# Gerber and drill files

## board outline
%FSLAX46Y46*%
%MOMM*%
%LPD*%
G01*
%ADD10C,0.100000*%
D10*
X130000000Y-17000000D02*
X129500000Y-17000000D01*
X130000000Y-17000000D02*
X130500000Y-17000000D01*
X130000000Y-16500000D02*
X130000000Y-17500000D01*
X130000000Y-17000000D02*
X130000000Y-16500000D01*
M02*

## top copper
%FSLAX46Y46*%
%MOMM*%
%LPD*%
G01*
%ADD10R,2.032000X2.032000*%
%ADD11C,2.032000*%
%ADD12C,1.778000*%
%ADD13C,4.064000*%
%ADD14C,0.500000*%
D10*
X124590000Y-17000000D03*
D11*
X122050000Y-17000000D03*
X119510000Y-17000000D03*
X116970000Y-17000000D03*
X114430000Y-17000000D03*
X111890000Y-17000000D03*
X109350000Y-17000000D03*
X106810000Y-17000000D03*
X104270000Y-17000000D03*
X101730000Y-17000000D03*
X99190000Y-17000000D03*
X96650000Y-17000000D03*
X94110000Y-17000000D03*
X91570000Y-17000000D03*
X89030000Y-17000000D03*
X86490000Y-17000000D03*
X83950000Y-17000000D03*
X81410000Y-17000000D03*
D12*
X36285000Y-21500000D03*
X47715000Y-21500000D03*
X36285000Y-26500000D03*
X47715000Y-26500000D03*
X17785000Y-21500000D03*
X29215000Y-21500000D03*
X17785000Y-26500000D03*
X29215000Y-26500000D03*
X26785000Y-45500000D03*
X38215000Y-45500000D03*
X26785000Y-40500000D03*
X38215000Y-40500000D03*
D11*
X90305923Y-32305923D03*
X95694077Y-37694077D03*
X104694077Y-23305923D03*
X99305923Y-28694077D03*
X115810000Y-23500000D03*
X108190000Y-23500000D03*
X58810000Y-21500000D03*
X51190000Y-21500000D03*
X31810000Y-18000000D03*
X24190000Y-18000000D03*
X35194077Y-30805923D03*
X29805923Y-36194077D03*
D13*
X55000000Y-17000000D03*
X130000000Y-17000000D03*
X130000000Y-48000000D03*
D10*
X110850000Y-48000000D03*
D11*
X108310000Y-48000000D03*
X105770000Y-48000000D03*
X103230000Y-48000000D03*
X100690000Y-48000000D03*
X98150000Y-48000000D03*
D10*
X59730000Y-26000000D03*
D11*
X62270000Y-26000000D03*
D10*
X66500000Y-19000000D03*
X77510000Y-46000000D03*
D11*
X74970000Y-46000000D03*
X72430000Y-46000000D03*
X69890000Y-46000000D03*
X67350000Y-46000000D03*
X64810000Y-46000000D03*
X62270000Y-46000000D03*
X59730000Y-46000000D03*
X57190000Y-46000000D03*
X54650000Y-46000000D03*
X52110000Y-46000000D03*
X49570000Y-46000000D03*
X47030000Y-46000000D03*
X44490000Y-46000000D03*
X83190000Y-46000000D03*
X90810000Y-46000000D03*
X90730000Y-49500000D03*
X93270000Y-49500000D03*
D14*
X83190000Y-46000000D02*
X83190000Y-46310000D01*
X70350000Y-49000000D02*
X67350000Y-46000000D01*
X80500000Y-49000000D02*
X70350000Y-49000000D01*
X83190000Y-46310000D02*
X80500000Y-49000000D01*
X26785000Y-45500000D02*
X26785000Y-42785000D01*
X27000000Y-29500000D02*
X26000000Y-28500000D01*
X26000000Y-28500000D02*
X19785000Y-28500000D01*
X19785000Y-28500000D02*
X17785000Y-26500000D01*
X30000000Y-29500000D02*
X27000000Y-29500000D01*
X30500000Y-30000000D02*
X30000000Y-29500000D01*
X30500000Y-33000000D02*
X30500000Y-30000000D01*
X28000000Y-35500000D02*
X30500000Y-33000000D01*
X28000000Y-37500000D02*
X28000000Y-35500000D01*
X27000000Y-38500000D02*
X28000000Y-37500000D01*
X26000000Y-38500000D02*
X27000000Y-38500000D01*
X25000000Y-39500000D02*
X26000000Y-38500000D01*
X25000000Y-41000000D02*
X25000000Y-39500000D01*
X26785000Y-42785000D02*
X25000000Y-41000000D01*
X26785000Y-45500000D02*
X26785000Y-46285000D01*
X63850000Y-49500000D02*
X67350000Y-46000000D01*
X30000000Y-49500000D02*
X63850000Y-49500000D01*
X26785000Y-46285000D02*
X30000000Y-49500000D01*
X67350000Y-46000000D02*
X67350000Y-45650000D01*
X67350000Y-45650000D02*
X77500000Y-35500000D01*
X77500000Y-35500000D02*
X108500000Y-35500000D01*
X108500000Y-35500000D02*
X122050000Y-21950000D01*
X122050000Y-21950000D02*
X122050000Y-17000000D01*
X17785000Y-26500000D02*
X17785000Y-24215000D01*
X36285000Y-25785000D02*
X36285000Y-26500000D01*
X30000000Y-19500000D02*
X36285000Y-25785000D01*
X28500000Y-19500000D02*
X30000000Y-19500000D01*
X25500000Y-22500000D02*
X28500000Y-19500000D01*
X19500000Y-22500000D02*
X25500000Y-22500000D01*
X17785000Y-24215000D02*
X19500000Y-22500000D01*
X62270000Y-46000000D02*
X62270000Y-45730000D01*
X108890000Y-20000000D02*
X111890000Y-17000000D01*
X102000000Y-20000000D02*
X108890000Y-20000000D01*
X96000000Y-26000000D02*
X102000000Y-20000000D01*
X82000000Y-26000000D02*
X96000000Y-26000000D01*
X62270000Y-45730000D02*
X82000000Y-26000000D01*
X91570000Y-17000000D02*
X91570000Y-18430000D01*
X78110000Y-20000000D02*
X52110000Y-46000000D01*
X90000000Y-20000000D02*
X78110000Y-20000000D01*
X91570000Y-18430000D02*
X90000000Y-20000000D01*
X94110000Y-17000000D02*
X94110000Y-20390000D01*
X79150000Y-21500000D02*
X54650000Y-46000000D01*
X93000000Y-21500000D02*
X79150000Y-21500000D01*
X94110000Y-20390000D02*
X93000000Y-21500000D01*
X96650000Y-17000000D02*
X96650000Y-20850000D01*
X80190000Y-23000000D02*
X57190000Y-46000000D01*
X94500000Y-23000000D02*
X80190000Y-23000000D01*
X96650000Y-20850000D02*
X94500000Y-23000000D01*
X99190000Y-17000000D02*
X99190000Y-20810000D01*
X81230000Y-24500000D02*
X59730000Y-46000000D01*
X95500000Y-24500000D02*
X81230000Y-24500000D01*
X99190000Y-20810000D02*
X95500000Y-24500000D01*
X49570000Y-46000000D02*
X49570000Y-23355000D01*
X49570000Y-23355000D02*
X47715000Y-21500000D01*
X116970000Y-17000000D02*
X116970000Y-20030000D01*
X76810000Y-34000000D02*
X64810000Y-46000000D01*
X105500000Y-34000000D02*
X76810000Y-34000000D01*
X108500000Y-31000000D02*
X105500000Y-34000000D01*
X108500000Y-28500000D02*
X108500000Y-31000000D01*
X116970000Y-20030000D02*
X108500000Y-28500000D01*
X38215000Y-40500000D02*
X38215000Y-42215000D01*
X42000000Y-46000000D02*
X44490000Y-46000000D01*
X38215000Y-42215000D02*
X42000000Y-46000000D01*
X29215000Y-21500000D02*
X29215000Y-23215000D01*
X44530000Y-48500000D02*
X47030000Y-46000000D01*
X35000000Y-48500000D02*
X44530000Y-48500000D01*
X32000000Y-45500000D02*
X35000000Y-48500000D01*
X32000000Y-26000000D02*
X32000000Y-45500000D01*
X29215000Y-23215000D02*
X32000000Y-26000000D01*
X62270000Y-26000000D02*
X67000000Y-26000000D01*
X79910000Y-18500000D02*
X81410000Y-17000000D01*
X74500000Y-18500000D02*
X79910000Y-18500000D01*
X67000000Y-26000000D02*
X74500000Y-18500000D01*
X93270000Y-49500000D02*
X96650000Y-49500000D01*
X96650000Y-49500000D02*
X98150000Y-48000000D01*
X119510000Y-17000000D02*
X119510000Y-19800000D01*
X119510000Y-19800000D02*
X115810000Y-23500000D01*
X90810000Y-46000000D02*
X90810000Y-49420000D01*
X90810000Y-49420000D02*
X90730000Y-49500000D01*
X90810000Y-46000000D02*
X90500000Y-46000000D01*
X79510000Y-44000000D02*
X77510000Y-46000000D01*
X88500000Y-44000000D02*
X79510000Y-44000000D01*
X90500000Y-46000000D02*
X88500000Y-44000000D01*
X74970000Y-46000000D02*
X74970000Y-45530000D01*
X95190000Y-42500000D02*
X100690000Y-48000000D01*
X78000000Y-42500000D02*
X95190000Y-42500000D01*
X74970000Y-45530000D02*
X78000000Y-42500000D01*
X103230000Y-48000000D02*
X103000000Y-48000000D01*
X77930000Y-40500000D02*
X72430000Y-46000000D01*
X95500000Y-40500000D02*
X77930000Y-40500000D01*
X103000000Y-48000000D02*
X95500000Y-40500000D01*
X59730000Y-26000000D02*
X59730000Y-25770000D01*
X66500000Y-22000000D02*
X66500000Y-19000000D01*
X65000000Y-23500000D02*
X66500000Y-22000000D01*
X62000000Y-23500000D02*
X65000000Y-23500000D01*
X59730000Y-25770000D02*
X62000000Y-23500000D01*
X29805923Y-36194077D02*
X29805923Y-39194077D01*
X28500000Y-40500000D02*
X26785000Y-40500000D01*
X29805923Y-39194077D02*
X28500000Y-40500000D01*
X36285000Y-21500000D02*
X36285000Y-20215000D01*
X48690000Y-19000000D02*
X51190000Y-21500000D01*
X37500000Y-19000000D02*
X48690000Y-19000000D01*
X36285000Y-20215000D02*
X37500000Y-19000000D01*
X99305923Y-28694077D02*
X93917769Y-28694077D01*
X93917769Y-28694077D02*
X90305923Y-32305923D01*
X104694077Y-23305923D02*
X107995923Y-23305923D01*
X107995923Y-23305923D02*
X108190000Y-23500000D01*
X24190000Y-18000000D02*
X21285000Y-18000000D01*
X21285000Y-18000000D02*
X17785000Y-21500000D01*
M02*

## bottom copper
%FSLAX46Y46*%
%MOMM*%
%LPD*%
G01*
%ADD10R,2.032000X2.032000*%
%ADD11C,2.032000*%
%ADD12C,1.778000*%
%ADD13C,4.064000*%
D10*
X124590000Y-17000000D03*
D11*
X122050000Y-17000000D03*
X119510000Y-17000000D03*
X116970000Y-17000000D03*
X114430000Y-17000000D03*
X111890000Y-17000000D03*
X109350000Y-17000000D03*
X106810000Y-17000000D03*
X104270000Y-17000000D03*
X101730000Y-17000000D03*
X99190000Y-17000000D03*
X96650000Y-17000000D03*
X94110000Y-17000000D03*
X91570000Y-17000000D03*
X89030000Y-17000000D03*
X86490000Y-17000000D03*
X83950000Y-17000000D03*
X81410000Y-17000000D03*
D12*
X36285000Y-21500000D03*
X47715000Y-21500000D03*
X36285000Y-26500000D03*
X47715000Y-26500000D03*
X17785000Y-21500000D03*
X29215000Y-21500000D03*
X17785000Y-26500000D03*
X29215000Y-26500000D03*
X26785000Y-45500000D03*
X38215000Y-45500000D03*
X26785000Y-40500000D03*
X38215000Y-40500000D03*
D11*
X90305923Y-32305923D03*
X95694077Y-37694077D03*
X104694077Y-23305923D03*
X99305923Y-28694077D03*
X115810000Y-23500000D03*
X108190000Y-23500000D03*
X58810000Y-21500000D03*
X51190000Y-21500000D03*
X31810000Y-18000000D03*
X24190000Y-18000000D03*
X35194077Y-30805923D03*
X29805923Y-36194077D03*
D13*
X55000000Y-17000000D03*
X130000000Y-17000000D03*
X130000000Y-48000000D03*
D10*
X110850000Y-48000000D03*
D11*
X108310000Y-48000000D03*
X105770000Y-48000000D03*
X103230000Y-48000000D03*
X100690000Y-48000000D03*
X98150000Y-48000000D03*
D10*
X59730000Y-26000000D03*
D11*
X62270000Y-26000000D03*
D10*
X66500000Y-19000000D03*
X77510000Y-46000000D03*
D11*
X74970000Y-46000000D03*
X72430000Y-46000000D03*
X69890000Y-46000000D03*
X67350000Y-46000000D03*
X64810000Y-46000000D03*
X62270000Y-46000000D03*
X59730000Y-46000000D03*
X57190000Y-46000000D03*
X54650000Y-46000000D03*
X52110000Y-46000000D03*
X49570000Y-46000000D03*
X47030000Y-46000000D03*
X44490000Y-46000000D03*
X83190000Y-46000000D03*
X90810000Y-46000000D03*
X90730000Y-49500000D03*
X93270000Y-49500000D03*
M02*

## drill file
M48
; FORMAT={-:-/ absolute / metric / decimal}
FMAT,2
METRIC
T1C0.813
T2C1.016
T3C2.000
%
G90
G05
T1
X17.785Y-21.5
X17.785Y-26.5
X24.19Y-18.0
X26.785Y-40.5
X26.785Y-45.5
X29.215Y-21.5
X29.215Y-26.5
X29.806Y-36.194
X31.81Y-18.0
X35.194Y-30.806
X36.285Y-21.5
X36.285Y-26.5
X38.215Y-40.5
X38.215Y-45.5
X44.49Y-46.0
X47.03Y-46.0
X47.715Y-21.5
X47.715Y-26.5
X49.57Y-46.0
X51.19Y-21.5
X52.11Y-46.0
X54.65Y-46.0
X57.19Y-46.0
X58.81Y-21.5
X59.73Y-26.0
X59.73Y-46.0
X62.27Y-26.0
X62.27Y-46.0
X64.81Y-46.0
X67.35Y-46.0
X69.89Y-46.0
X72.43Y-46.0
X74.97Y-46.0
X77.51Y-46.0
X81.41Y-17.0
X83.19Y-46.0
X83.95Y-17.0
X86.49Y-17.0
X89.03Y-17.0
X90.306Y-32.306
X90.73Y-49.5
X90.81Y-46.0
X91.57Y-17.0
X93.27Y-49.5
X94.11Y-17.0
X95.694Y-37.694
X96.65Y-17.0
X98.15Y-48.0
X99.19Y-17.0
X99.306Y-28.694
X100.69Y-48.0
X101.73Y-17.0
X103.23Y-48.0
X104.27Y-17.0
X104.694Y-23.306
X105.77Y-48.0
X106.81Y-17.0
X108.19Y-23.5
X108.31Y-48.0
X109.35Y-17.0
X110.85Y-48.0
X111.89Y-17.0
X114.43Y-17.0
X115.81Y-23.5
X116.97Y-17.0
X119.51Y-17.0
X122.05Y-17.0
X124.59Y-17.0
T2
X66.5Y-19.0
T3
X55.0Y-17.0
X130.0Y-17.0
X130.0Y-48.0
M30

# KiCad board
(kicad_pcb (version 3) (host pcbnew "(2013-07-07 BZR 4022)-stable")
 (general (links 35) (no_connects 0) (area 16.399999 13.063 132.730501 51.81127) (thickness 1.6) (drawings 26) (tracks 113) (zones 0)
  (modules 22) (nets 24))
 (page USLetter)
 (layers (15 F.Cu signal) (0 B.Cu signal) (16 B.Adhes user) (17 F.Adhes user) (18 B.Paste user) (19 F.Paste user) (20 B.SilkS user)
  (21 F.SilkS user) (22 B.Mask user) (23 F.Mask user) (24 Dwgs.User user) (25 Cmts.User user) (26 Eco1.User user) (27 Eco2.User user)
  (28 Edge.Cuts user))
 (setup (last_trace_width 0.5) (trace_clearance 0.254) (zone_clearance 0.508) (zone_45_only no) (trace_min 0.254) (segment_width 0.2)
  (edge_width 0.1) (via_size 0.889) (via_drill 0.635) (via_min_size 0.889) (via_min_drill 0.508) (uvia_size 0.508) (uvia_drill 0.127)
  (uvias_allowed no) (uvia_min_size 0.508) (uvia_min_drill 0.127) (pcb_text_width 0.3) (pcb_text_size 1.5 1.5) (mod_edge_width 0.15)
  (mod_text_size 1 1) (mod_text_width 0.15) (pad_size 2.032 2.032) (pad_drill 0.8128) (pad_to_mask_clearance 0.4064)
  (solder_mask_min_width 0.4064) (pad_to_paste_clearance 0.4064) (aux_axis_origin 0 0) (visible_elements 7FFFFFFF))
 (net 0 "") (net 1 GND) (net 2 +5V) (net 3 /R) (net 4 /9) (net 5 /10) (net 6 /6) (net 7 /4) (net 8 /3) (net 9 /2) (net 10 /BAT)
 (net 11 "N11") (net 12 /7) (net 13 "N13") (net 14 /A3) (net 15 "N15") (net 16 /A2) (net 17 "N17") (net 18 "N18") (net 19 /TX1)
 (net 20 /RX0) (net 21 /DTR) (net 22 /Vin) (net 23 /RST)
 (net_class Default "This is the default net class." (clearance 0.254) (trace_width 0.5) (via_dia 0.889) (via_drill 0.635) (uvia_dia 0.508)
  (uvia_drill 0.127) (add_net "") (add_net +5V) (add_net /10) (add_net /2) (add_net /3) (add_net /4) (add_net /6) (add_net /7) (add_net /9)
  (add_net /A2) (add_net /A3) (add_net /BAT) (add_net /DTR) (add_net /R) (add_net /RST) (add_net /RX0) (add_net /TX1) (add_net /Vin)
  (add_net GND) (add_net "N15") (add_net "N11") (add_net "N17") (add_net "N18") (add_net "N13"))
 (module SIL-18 (layer F.Cu) (at 103 17 180) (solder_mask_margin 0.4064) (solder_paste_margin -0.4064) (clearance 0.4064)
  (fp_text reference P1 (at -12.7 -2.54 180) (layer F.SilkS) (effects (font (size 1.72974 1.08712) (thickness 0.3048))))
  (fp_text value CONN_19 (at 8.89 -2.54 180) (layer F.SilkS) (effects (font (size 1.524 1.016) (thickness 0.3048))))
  (pad 1 thru_hole rect (at -21.59 0 180) (size 2.032 2.032) (drill 0.8128) (layers *.Cu *.Mask F.SilkS) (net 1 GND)
   (solder_mask_margin 0.4064) (solder_paste_margin -0.4064) (clearance 0.4064) (thermal_width 0.508) (thermal_gap 0.508))
  (pad 2 thru_hole circle (at -19.05 0 180) (size 2.032 2.032) (drill 0.8128) (layers *.Cu *.Mask F.SilkS) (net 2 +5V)
   (solder_mask_margin 0.4064) (solder_paste_margin -0.4064))
  (pad 3 thru_hole circle (at -16.51 0 180) (size 2.032 2.032) (drill 0.8128) (layers *.Cu *.Mask F.SilkS) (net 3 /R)
   (solder_mask_margin 0.4064) (solder_paste_margin -0.4064))
  (pad 4 thru_hole circle (at -13.97 0 180) (size 2.032 2.032) (drill 0.8128) (layers *.Cu *.Mask F.SilkS) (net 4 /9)
   (solder_mask_margin 0.4064) (solder_paste_margin -0.4064))
  (pad 5 thru_hole circle (at -11.43 0 180) (size 2.032 2.032) (drill 0.8128) (layers *.Cu *.Mask F.SilkS) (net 1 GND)
   (solder_mask_margin 0.4064) (solder_paste_margin -0.4064))
  (pad 6 thru_hole circle (at -8.89 0 180) (size 2.032 2.032) (drill 0.8128) (layers *.Cu *.Mask F.SilkS) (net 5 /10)
   (solder_mask_margin 0.4064) (solder_paste_margin -0.4064) (clearance 0.4064) (thermal_width 0.508) (thermal_gap 0.508))
  (pad 7 thru_hole circle (at -6.35 0 180) (size 2.032 2.032) (drill 0.8128) (layers *.Cu *.Mask F.SilkS) (solder_mask_margin 0.4064)
   (solder_paste_margin -0.4064))
  (pad 8 thru_hole circle (at -3.81 0 180) (size 2.032 2.032) (drill 0.8128) (layers *.Cu *.Mask F.SilkS) (solder_mask_margin 0.4064)
   (solder_paste_margin -0.4064))
  (pad 9 thru_hole circle (at -1.27 0 180) (size 2.032 2.032) (drill 0.8128) (layers *.Cu *.Mask F.SilkS) (solder_mask_margin 0.4064)
   (solder_paste_margin -0.4064))
  (pad 10 thru_hole circle (at 1.27 0 180) (size 2.032 2.032) (drill 0.8128) (layers *.Cu *.Mask F.SilkS) (solder_mask_margin 0.4064)
   (solder_paste_margin -0.4064) (clearance 0.4064) (thermal_width 0.508) (thermal_gap 0.508))
  (pad 11 thru_hole circle (at 3.81 0 180) (size 2.032 2.032) (drill 0.8128) (layers *.Cu *.Mask F.SilkS) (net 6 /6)
   (solder_mask_margin 0.4064) (solder_paste_margin -0.4064) (clearance 0.4064) (thermal_width 0.508) (thermal_gap 0.508))
  (pad 12 thru_hole circle (at 6.35 0 180) (size 2.032 2.032) (drill 0.8128) (layers *.Cu *.Mask F.SilkS) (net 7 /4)
   (solder_mask_margin 0.4064) (solder_paste_margin -0.4064))
  (pad 13 thru_hole circle (at 8.89 0 180) (size 2.032 2.032) (drill 0.8128) (layers *.Cu *.Mask F.SilkS) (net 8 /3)
   (solder_mask_margin 0.4064) (solder_paste_margin -0.4064))
  (pad 14 thru_hole circle (at 11.43 0 180) (size 2.032 2.032) (drill 0.8128) (layers *.Cu *.Mask F.SilkS) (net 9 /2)
   (solder_mask_margin 0.4064) (solder_paste_margin -0.4064) (clearance 0.4064) (thermal_width 0.508) (thermal_gap 0.508))
  (pad 15 thru_hole circle (at 13.97 0 180) (size 2.032 2.032) (drill 0.8128) (layers *.Cu *.Mask F.SilkS) (solder_mask_margin 0.4064)
   (solder_paste_margin -0.4064))
  (pad 16 thru_hole circle (at 16.51 0 180) (size 2.032 2.032) (drill 0.8128) (layers *.Cu *.Mask F.SilkS) (solder_mask_margin 0.4064)
   (solder_paste_margin -0.4064))
  (pad 17 thru_hole circle (at 19.05 0 180) (size 2.032 2.032) (drill 0.8128) (layers *.Cu *.Mask F.SilkS) (solder_mask_margin 0.4064)
   (solder_paste_margin -0.4064) (clearance 0.4064) (thermal_width 0.508) (thermal_gap 0.508))
  (pad 18 thru_hole circle (at 21.59 0 180) (size 2.032 2.032) (drill 0.8128) (layers *.Cu *.Mask F.SilkS) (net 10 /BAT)
   (solder_mask_margin 0.4064) (solder_paste_margin -0.4064) (clearance 0.4064) (thermal_width 0.508) (thermal_gap 0.508)))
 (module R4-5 (layer F.Cu) (at 42 21.5)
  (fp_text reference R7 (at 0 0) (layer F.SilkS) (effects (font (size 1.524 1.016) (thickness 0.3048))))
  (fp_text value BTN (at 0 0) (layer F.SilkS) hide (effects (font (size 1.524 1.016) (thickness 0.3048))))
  (pad 1 thru_hole circle (at -5.715 0) (size 1.778 1.778) (drill 0.8128) (layers *.Cu *.Mask F.SilkS) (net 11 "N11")
   (solder_mask_margin 0.4064) (solder_paste_margin -0.4064))
  (pad 2 thru_hole circle (at 5.715 0) (size 1.778 1.778) (drill 0.8128) (layers *.Cu *.Mask F.SilkS) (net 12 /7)
   (solder_mask_margin 0.4064) (solder_paste_margin -0.4064)))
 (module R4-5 (layer F.Cu) (at 42 26.5)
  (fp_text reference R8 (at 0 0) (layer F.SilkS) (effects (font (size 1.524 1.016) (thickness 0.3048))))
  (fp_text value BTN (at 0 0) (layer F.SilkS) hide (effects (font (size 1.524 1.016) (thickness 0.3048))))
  (pad 1 thru_hole circle (at -5.715 0) (size 1.778 1.778) (drill 0.8128) (layers *.Cu *.Mask F.SilkS) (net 2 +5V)
   (solder_mask_margin 0.4064) (solder_paste_margin -0.4064))
  (pad 2 thru_hole circle (at 5.715 0) (size 1.778 1.778) (drill 0.8128) (layers *.Cu *.Mask F.SilkS) (solder_mask_margin 0.4064)
   (solder_paste_margin -0.4064) (clearance 0.4064) (thermal_width 0.508) (thermal_gap 0.508)))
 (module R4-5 (layer F.Cu) (at 23.5 21.5)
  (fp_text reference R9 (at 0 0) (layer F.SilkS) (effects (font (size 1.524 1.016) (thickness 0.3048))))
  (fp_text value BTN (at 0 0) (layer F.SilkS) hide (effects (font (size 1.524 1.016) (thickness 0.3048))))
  (pad 1 thru_hole circle (at -5.715 0) (size 1.778 1.778) (drill 0.8128) (layers *.Cu *.Mask F.SilkS) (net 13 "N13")
   (solder_mask_margin 0.4064) (solder_paste_margin -0.4064))
  (pad 2 thru_hole circle (at 5.715 0) (size 1.778 1.778) (drill 0.8128) (layers *.Cu *.Mask F.SilkS) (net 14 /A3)
   (solder_mask_margin 0.4064) (solder_paste_margin -0.4064)))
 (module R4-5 (layer F.Cu) (at 23.5 26.5)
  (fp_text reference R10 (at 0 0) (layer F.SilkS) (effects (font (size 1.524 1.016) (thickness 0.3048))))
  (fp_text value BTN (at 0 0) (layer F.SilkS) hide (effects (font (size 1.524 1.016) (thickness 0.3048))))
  (pad 1 thru_hole circle (at -5.715 0) (size 1.778 1.778) (drill 0.8128) (layers *.Cu *.Mask F.SilkS) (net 2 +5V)
   (solder_mask_margin 0.4064) (solder_paste_margin -0.4064))
  (pad 2 thru_hole circle (at 5.715 0) (size 1.778 1.778) (drill 0.8128) (layers *.Cu *.Mask F.SilkS) (solder_mask_margin 0.4064)
   (solder_paste_margin -0.4064)))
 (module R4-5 (layer F.Cu) (at 32.5 45.5)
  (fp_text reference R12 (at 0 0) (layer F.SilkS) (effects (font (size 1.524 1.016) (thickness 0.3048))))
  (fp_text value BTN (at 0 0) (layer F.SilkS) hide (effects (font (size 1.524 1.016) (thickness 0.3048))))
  (pad 1 thru_hole circle (at -5.715 0) (size 1.778 1.778) (drill 0.8128) (layers *.Cu *.Mask F.SilkS) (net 2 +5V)
   (solder_mask_margin 0.4064) (solder_paste_margin -0.4064))
  (pad 2 thru_hole circle (at 5.715 0) (size 1.778 1.778) (drill 0.8128) (layers *.Cu *.Mask F.SilkS) (solder_mask_margin 0.4064)
   (solder_paste_margin -0.4064)))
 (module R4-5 (layer F.Cu) (at 32.5 40.5)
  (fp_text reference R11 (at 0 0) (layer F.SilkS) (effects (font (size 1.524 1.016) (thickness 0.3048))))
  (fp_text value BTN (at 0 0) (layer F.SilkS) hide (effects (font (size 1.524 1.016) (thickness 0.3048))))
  (pad 1 thru_hole circle (at -5.715 0) (size 1.778 1.778) (drill 0.8128) (layers *.Cu *.Mask F.SilkS) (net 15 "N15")
   (solder_mask_margin 0.4064) (solder_paste_margin -0.4064))
  (pad 2 thru_hole circle (at 5.715 0) (size 1.778 1.778) (drill 0.8128) (layers *.Cu *.Mask F.SilkS) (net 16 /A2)
   (solder_mask_margin 0.4064) (solder_paste_margin -0.4064)))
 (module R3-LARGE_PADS (layer F.Cu) (at 93 35 315) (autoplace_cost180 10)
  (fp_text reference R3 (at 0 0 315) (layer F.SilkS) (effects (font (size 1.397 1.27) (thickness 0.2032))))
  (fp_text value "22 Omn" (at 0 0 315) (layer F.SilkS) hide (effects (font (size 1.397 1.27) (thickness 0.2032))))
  (pad 1 thru_hole circle (at -3.81 0 315) (size 2.032 2.032) (drill 0.8128) (layers *.Cu *.Mask F.SilkS) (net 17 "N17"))
  (pad 2 thru_hole circle (at 3.81 0 315) (size 2.032 2.032) (drill 0.8128) (layers *.Cu *.Mask F.SilkS) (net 1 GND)))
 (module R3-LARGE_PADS (layer F.Cu) (at 102 26 225) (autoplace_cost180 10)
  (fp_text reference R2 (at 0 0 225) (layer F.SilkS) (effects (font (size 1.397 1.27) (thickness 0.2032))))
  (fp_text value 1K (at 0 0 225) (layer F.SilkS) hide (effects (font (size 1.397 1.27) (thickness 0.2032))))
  (pad 1 thru_hole circle (at -3.81 0 225) (size 2.032 2.032) (drill 0.8128) (layers *.Cu *.Mask F.SilkS) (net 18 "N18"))
  (pad 2 thru_hole circle (at 3.81 0 225) (size 2.032 2.032) (drill 0.8128) (layers *.Cu *.Mask F.SilkS) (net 17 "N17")))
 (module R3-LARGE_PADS (layer F.Cu) (at 112 23.5 180) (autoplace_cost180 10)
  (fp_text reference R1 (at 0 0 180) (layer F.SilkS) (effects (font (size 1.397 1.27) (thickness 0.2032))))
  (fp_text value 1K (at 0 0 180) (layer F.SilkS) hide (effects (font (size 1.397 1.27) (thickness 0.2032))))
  (pad 1 thru_hole circle (at -3.81 0 180) (size 2.032 2.032) (drill 0.8128) (layers *.Cu *.Mask F.SilkS) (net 3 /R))
  (pad 2 thru_hole circle (at 3.81 0 180) (size 2.032 2.032) (drill 0.8128) (layers *.Cu *.Mask F.SilkS) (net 18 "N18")))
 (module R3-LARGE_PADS (layer F.Cu) (at 55 21.5 180) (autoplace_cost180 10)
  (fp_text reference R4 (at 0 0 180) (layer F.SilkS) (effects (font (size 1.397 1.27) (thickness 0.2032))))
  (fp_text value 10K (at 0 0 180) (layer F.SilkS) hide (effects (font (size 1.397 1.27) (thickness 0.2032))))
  (pad 1 thru_hole circle (at -3.81 0 180) (size 2.032 2.032) (drill 0.8128) (layers *.Cu *.Mask F.SilkS) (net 1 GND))
  (pad 2 thru_hole circle (at 3.81 0 180) (size 2.032 2.032) (drill 0.8128) (layers *.Cu *.Mask F.SilkS) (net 11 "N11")))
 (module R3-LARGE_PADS (layer F.Cu) (at 28 18 180) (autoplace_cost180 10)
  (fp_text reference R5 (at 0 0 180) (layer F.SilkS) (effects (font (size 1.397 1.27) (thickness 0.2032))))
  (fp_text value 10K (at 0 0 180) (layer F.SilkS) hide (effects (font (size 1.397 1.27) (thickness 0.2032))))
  (pad 1 thru_hole circle (at -3.81 0 180) (size 2.032 2.032) (drill 0.8128) (layers *.Cu *.Mask F.SilkS) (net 1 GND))
  (pad 2 thru_hole circle (at 3.81 0 180) (size 2.032 2.032) (drill 0.8128) (layers *.Cu *.Mask F.SilkS) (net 13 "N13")))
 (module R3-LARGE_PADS (layer F.Cu) (at 32.5 33.5 225) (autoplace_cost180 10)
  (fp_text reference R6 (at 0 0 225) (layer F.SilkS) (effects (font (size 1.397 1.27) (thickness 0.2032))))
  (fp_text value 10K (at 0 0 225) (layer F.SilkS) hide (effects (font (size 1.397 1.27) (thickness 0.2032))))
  (pad 1 thru_hole circle (at -3.81 0 225) (size 2.032 2.032) (drill 0.8128) (layers *.Cu *.Mask F.SilkS) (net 1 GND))
  (pad 2 thru_hole circle (at 3.81 0 225) (size 2.032 2.032) (drill 0.8128) (layers *.Cu *.Mask F.SilkS) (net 15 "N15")))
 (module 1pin (layer F.Cu) (at 55 17)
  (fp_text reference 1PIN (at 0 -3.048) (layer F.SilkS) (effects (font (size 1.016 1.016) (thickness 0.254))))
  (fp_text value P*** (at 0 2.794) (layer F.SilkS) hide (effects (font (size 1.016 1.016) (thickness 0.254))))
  (pad 1 thru_hole circle (at 0 0) (size 4.064 4.064) (drill 2) (layers *.Cu *.Mask F.SilkS)))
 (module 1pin (layer F.Cu) (at 130 17)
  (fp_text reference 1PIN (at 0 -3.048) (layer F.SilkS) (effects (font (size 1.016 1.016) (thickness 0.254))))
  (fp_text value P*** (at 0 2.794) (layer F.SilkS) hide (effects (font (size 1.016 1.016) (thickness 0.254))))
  (pad 1 thru_hole circle (at 0 0) (size 4.064 4.064) (drill 2) (layers *.Cu *.Mask F.SilkS)))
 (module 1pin (layer F.Cu) (at 130 48)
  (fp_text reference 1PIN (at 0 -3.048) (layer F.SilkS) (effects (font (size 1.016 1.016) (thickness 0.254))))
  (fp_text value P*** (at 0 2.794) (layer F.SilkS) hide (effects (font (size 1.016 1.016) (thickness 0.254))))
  (pad 1 thru_hole circle (at 0 0) (size 4.064 4.064) (drill 2) (layers *.Cu *.Mask F.SilkS)))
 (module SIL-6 (layer F.Cu) (at 104.5 48 180)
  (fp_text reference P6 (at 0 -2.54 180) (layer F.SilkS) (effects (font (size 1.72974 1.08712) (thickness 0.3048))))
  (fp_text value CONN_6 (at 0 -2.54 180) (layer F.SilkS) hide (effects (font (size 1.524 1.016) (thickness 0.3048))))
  (pad 1 thru_hole rect (at -6.35 0 180) (size 2.032 2.032) (drill 0.8128) (layers *.Cu *.Mask F.SilkS) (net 1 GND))
  (pad 2 thru_hole circle (at -3.81 0 180) (size 2.032 2.032) (drill 0.8128) (layers *.Cu *.Mask F.SilkS) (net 1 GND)
   (solder_mask_margin 0.4064) (solder_paste_margin -0.4064))
  (pad 3 thru_hole circle (at -1.27 0 180) (size 2.032 2.032) (drill 0.8128) (layers *.Cu *.Mask F.SilkS) (solder_mask_margin 0.4064)
   (solder_paste_margin -0.4064) (clearance 0.4064) (thermal_width 0.508) (thermal_gap 0.508))
  (pad 4 thru_hole circle (at 1.27 0 180) (size 2.032 2.032) (drill 0.8128) (layers *.Cu *.Mask F.SilkS) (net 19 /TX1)
   (solder_mask_margin 0.4064) (solder_paste_margin -0.4064))
  (pad 5 thru_hole circle (at 3.81 0 180) (size 2.032 2.032) (drill 0.8128) (layers *.Cu *.Mask F.SilkS) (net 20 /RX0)
   (solder_mask_margin 0.4064) (solder_paste_margin -0.4064))
  (pad 6 thru_hole circle (at 6.35 0 180) (size 2.032 2.032) (drill 0.8128) (layers *.Cu *.Mask F.SilkS) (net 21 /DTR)
   (solder_mask_margin 0.4064) (solder_paste_margin -0.4064)))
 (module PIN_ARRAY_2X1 (layer F.Cu) (at 61 26)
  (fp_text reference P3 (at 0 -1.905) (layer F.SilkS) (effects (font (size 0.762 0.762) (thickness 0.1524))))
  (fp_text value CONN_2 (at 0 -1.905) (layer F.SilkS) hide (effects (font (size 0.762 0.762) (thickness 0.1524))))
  (pad 1 thru_hole rect (at -1.27 0) (size 2.032 2.032) (drill 0.8128) (layers *.Cu *.Mask F.SilkS) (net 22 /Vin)
   (solder_mask_margin 0.4064) (solder_paste_margin -0.4064) (clearance 0.4064) (thermal_width 0.508) (thermal_gap 0.508))
  (pad 2 thru_hole circle (at 1.27 0) (size 2.032 2.032) (drill 0.8128) (layers *.Cu *.Mask F.SilkS) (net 10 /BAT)
   (solder_mask_margin 0.4064) (solder_paste_margin -0.4064) (clearance 0.4064) (thermal_width 0.508) (thermal_gap 0.508)))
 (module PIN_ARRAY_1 (layer F.Cu) (at 66.5 19)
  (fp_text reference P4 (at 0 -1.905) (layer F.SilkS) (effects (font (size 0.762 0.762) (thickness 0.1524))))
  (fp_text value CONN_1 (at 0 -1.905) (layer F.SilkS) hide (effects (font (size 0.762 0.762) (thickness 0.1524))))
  (pad 1 thru_hole rect (at 0 0) (size 2.032 2.032) (drill 1.016) (layers *.Cu *.Mask F.SilkS) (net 22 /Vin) (solder_mask_margin 0.4064)
   (solder_paste_margin -0.4064) (clearance 0.4064) (thermal_width 0.508) (thermal_gap 0.508)))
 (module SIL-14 (layer F.Cu) (at 61 46 180)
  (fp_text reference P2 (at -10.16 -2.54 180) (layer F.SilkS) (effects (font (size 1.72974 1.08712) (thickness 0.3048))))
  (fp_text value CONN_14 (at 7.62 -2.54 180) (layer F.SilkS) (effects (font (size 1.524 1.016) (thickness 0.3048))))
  (pad 1 thru_hole rect (at -16.51 0 180) (size 2.032 2.032) (drill 0.8128) (layers *.Cu *.Mask F.SilkS) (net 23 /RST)
   (solder_mask_margin 0.4064) (solder_paste_margin -0.4064) (clearance 0.4064) (thermal_width 0.508) (thermal_gap 0.508))
  (pad 2 thru_hole circle (at -13.97 0 180) (size 2.032 2.032) (drill 0.8128) (layers *.Cu *.Mask F.SilkS) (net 20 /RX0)
   (solder_mask_margin 0.4064) (solder_paste_margin -0.4064) (clearance 0.4064) (thermal_width 0.508) (thermal_gap 0.508))
  (pad 3 thru_hole circle (at -11.43 0 180) (size 2.032 2.032) (drill 0.8128) (layers *.Cu *.Mask F.SilkS) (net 19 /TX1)
   (solder_mask_margin 0.4064) (solder_paste_margin -0.4064))
  (pad 4 thru_hole circle (at -8.89 0 180) (size 2.032 2.032) (drill 0.8128) (layers *.Cu *.Mask F.SilkS) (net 1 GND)
   (solder_mask_margin 0.4064) (solder_paste_margin -0.4064) (clearance 0.4064) (thermal_width 0.508) (thermal_gap 0.508))
  (pad 5 thru_hole circle (at -6.35 0 180) (size 2.032 2.032) (drill 0.8128) (layers *.Cu *.Mask F.SilkS) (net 2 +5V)
   (solder_mask_margin 0.4064) (solder_paste_margin -0.4064))
  (pad 6 thru_hole circle (at -3.81 0 180) (size 2.032 2.032) (drill 0.8128) (layers *.Cu *.Mask F.SilkS) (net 4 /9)
   (solder_mask_margin 0.4064) (solder_paste_margin -0.4064))
  (pad 7 thru_hole circle (at -1.27 0 180) (size 2.032 2.032) (drill 0.8128) (layers *.Cu *.Mask F.SilkS) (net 5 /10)
   (solder_mask_margin 0.4064) (solder_paste_margin -0.4064))
  (pad 8 thru_hole circle (at 1.27 0 180) (size 2.032 2.032) (drill 0.8128) (layers *.Cu *.Mask F.SilkS) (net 6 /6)
   (solder_mask_margin 0.4064) (solder_paste_margin -0.4064))
  (pad 9 thru_hole circle (at 3.81 0 180) (size 2.032 2.032) (drill 0.8128) (layers *.Cu *.Mask F.SilkS) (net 7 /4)
   (solder_mask_margin 0.4064) (solder_paste_margin -0.4064))
  (pad 10 thru_hole circle (at 6.35 0 180) (size 2.032 2.032) (drill 0.8128) (layers *.Cu *.Mask F.SilkS) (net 8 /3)
   (solder_mask_margin 0.4064) (solder_paste_margin -0.4064))
  (pad 11 thru_hole circle (at 8.89 0 180) (size 2.032 2.032) (drill 0.8128) (layers *.Cu *.Mask F.SilkS) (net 9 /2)
   (solder_mask_margin 0.4064) (solder_paste_margin -0.4064))
  (pad 12 thru_hole circle (at 11.43 0 180) (size 2.032 2.032) (drill 0.8128) (layers *.Cu *.Mask F.SilkS) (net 12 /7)
   (solder_mask_margin 0.4064) (solder_paste_margin -0.4064))
  (pad 13 thru_hole circle (at 13.97 0 180) (size 2.032 2.032) (drill 0.8128) (layers *.Cu *.Mask F.SilkS) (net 14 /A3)
   (solder_mask_margin 0.4064) (solder_paste_margin -0.4064))
  (pad 14 thru_hole circle (at 16.51 0 180) (size 2.032 2.032) (drill 0.8128) (layers *.Cu *.Mask F.SilkS) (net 16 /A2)
   (solder_mask_margin 0.4064) (solder_paste_margin -0.4064)))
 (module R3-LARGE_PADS (layer F.Cu) (at 87 46) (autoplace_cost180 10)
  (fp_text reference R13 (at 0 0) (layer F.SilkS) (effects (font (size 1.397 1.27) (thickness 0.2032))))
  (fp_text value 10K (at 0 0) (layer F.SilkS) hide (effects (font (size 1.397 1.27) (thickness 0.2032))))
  (pad 1 thru_hole circle (at -3.81 0) (size 2.032 2.032) (drill 0.8128) (layers *.Cu *.Mask F.SilkS) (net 2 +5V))
  (pad 2 thru_hole circle (at 3.81 0) (size 2.032 2.032) (drill 0.8128) (layers *.Cu *.Mask F.SilkS) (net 23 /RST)))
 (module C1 (layer F.Cu) (at 92 49.5)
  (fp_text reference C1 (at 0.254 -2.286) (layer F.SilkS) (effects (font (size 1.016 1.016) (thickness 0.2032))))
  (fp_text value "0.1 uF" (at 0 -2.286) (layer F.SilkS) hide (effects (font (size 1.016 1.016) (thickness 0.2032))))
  (pad 1 thru_hole circle (at -1.27 0) (size 2.032 2.032) (drill 0.8128) (layers *.Cu *.Mask F.SilkS) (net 23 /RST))
  (pad 2 thru_hole circle (at 1.27 0) (size 2.032 2.032) (drill 0.8128) (layers *.Cu *.Mask F.SilkS) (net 21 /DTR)))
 (gr_line (start 130 17) (end 129.5 17) (angle 90) (layer Edge.Cuts) (width 0.1))
 (gr_line (start 130 17) (end 130.5 17) (angle 90) (layer Edge.Cuts) (width 0.1))
 (gr_line (start 130 16.5) (end 130 17.5) (angle 90) (layer Edge.Cuts) (width 0.1))
 (gr_line (start 130 17) (end 130 16.5) (angle 90) (layer Edge.Cuts) (width 0.1))
 (segment (start 83.19 46) (end 83.19 46.31) (width 0.5) (layer F.Cu) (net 2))
 (segment (start 70.35 49) (end 67.35 46) (width 0.5) (layer F.Cu) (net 2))
 (segment (start 80.5 49) (end 70.35 49) (width 0.5) (layer F.Cu) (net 2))
 (segment (start 83.19 46.31) (end 80.5 49) (width 0.5) (layer F.Cu) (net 2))
 (segment (start 26.785 45.5) (end 26.785 42.785) (width 0.5) (layer F.Cu) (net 2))
 (segment (start 27 29.5) (end 26 28.5) (width 0.5) (layer F.Cu) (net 2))
 (segment (start 26 28.5) (end 19.785 28.5) (width 0.5) (layer F.Cu) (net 2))
 (segment (start 19.785 28.5) (end 17.785 26.5) (width 0.5) (layer F.Cu) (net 2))
 (segment (start 30 29.5) (end 27 29.5) (width 0.5) (layer F.Cu) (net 2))
 (segment (start 30.5 30) (end 30 29.5) (width 0.5) (layer F.Cu) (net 2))
 (segment (start 30.5 33) (end 30.5 30) (width 0.5) (layer F.Cu) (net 2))
 (segment (start 28 35.5) (end 30.5 33) (width 0.5) (layer F.Cu) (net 2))
 (segment (start 28 37.5) (end 28 35.5) (width 0.5) (layer F.Cu) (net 2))
 (segment (start 27 38.5) (end 28 37.5) (width 0.5) (layer F.Cu) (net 2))
 (segment (start 26 38.5) (end 27 38.5) (width 0.5) (layer F.Cu) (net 2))
 (segment (start 25 39.5) (end 26 38.5) (width 0.5) (layer F.Cu) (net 2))
 (segment (start 25 41) (end 25 39.5) (width 0.5) (layer F.Cu) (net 2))
 (segment (start 26.785 42.785) (end 25 41) (width 0.5) (layer F.Cu) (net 2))
 (segment (start 26.785 45.5) (end 26.785 46.285) (width 0.5) (layer F.Cu) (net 2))
 (segment (start 63.85 49.5) (end 67.35 46) (width 0.5) (layer F.Cu) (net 2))
 (segment (start 30 49.5) (end 63.85 49.5) (width 0.5) (layer F.Cu) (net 2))
 (segment (start 26.785 46.285) (end 30 49.5) (width 0.5) (layer F.Cu) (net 2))
 (segment (start 67.35 46) (end 67.35 45.65) (width 0.5) (layer F.Cu) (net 2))
 (segment (start 67.35 45.65) (end 77.5 35.5) (width 0.5) (layer F.Cu) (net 2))
 (segment (start 77.5 35.5) (end 108.5 35.5) (width 0.5) (layer F.Cu) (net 2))
 (segment (start 108.5 35.5) (end 122.05 21.95) (width 0.5) (layer F.Cu) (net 2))
 (segment (start 122.05 21.95) (end 122.05 17) (width 0.5) (layer F.Cu) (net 2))
 (segment (start 17.785 26.5) (end 17.785 24.215) (width 0.5) (layer F.Cu) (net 2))
 (segment (start 36.285 25.785) (end 36.285 26.5) (width 0.5) (layer F.Cu) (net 2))
 (segment (start 30 19.5) (end 36.285 25.785) (width 0.5) (layer F.Cu) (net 2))
 (segment (start 28.5 19.5) (end 30 19.5) (width 0.5) (layer F.Cu) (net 2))
 (segment (start 25.5 22.5) (end 28.5 19.5) (width 0.5) (layer F.Cu) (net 2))
 (segment (start 19.5 22.5) (end 25.5 22.5) (width 0.5) (layer F.Cu) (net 2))
 (segment (start 17.785 24.215) (end 19.5 22.5) (width 0.5) (layer F.Cu) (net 2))
 (segment (start 62.27 46) (end 62.27 45.73) (width 0.5) (layer F.Cu) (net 5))
 (segment (start 108.89 20) (end 111.89 17) (width 0.5) (layer F.Cu) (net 5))
 (segment (start 102 20) (end 108.89 20) (width 0.5) (layer F.Cu) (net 5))
 (segment (start 96 26) (end 102 20) (width 0.5) (layer F.Cu) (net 5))
 (segment (start 82 26) (end 96 26) (width 0.5) (layer F.Cu) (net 5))
 (segment (start 62.27 45.73) (end 82 26) (width 0.5) (layer F.Cu) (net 5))
 (segment (start 91.57 17) (end 91.57 18.43) (width 0.5) (layer F.Cu) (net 9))
 (segment (start 78.11 20) (end 52.11 46) (width 0.5) (layer F.Cu) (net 9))
 (segment (start 90 20) (end 78.11 20) (width 0.5) (layer F.Cu) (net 9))
 (segment (start 91.57 18.43) (end 90 20) (width 0.5) (layer F.Cu) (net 9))
 (segment (start 94.11 17) (end 94.11 20.39) (width 0.5) (layer F.Cu) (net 8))
 (segment (start 79.15 21.5) (end 54.65 46) (width 0.5) (layer F.Cu) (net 8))
 (segment (start 93 21.5) (end 79.15 21.5) (width 0.5) (layer F.Cu) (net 8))
 (segment (start 94.11 20.39) (end 93 21.5) (width 0.5) (layer F.Cu) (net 8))
 (segment (start 96.65 17) (end 96.65 20.85) (width 0.5) (layer F.Cu) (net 7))
 (segment (start 80.19 23) (end 57.19 46) (width 0.5) (layer F.Cu) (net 7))
 (segment (start 94.5 23) (end 80.19 23) (width 0.5) (layer F.Cu) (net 7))
 (segment (start 96.65 20.85) (end 94.5 23) (width 0.5) (layer F.Cu) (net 7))
 (segment (start 99.19 17) (end 99.19 20.81) (width 0.5) (layer F.Cu) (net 6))
 (segment (start 81.23 24.5) (end 59.73 46) (width 0.5) (layer F.Cu) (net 6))
 (segment (start 95.5 24.5) (end 81.23 24.5) (width 0.5) (layer F.Cu) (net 6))
 (segment (start 99.19 20.81) (end 95.5 24.5) (width 0.5) (layer F.Cu) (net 6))
 (segment (start 49.57 46) (end 49.57 23.355) (width 0.5) (layer F.Cu) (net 12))
 (segment (start 49.57 23.355) (end 47.715 21.5) (width 0.5) (layer F.Cu) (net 12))
 (segment (start 116.97 17) (end 116.97 20.03) (width 0.5) (layer F.Cu) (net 4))
 (segment (start 76.81 34) (end 64.81 46) (width 0.5) (layer F.Cu) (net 4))
 (segment (start 105.5 34) (end 76.81 34) (width 0.5) (layer F.Cu) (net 4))
 (segment (start 108.5 31) (end 105.5 34) (width 0.5) (layer F.Cu) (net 4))
 (segment (start 108.5 28.5) (end 108.5 31) (width 0.5) (layer F.Cu) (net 4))
 (segment (start 116.97 20.03) (end 108.5 28.5) (width 0.5) (layer F.Cu) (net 4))
 (segment (start 38.215 40.5) (end 38.215 42.215) (width 0.5) (layer F.Cu) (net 16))
 (segment (start 42 46) (end 44.49 46) (width 0.5) (layer F.Cu) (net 16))
 (segment (start 38.215 42.215) (end 42 46) (width 0.5) (layer F.Cu) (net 16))
 (segment (start 29.215 21.5) (end 29.215 23.215) (width 0.5) (layer F.Cu) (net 14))
 (segment (start 44.53 48.5) (end 47.03 46) (width 0.5) (layer F.Cu) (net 14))
 (segment (start 35 48.5) (end 44.53 48.5) (width 0.5) (layer F.Cu) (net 14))
 (segment (start 32 45.5) (end 35 48.5) (width 0.5) (layer F.Cu) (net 14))
 (segment (start 32 26) (end 32 45.5) (width 0.5) (layer F.Cu) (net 14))
 (segment (start 29.215 23.215) (end 32 26) (width 0.5) (layer F.Cu) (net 14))
 (segment (start 62.27 26) (end 67 26) (width 0.5) (layer F.Cu) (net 10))
 (segment (start 79.91 18.5) (end 81.41 17) (width 0.5) (layer F.Cu) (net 10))
 (segment (start 74.5 18.5) (end 79.91 18.5) (width 0.5) (layer F.Cu) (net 10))
 (segment (start 67 26) (end 74.5 18.5) (width 0.5) (layer F.Cu) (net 10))
 (segment (start 93.27 49.5) (end 96.65 49.5) (width 0.5) (layer F.Cu) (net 21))
 (segment (start 96.65 49.5) (end 98.15 48) (width 0.5) (layer F.Cu) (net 21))
 (segment (start 119.51 17) (end 119.51 19.8) (width 0.5) (layer F.Cu) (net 3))
 (segment (start 119.51 19.8) (end 115.81 23.5) (width 0.5) (layer F.Cu) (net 3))
 (segment (start 90.81 46) (end 90.81 49.42) (width 0.5) (layer F.Cu) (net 23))
 (segment (start 90.81 49.42) (end 90.73 49.5) (width 0.5) (layer F.Cu) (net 23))
 (segment (start 90.81 46) (end 90.5 46) (width 0.5) (layer F.Cu) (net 23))
 (segment (start 79.51 44) (end 77.51 46) (width 0.5) (layer F.Cu) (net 23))
 (segment (start 88.5 44) (end 79.51 44) (width 0.5) (layer F.Cu) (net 23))
 (segment (start 90.5 46) (end 88.5 44) (width 0.5) (layer F.Cu) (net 23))
 (segment (start 74.97 46) (end 74.97 45.53) (width 0.5) (layer F.Cu) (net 20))
 (segment (start 95.19 42.5) (end 100.69 48) (width 0.5) (layer F.Cu) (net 20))
 (segment (start 78 42.5) (end 95.19 42.5) (width 0.5) (layer F.Cu) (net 20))
 (segment (start 74.97 45.53) (end 78 42.5) (width 0.5) (layer F.Cu) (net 20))
 (segment (start 103.23 48) (end 103 48) (width 0.5) (layer F.Cu) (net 19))
 (segment (start 77.93 40.5) (end 72.43 46) (width 0.5) (layer F.Cu) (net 19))
 (segment (start 95.5 40.5) (end 77.93 40.5) (width 0.5) (layer F.Cu) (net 19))
 (segment (start 103 48) (end 95.5 40.5) (width 0.5) (layer F.Cu) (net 19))
 (segment (start 59.73 26) (end 59.73 25.77) (width 0.5) (layer F.Cu) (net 22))
 (segment (start 66.5 22) (end 66.5 19) (width 0.5) (layer F.Cu) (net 22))
 (segment (start 65 23.5) (end 66.5 22) (width 0.5) (layer F.Cu) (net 22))
 (segment (start 62 23.5) (end 65 23.5) (width 0.5) (layer F.Cu) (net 22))
 (segment (start 59.73 25.77) (end 62 23.5) (width 0.5) (layer F.Cu) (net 22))
 (segment (start 29.805923 36.194077) (end 29.805923 39.194077) (width 0.5) (layer F.Cu) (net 15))
 (segment (start 28.5 40.5) (end 26.785 40.5) (width 0.5) (layer F.Cu) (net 15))
 (segment (start 29.805923 39.194077) (end 28.5 40.5) (width 0.5) (layer F.Cu) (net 15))
 (segment (start 36.285 21.5) (end 36.285 20.215) (width 0.5) (layer F.Cu) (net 11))
 (segment (start 48.69 19) (end 51.19 21.5) (width 0.5) (layer F.Cu) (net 11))
 (segment (start 37.5 19) (end 48.69 19) (width 0.5) (layer F.Cu) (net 11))
 (segment (start 36.285 20.215) (end 37.5 19) (width 0.5) (layer F.Cu) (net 11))
 (segment (start 99.305923 28.694077) (end 93.917769 28.694077) (width 0.5) (layer F.Cu) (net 17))
 (segment (start 93.917769 28.694077) (end 90.305923 32.305923) (width 0.5) (layer F.Cu) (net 17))
 (segment (start 104.694077 23.305923) (end 107.995923 23.305923) (width 0.5) (layer F.Cu) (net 18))
 (segment (start 107.995923 23.305923) (end 108.19 23.5) (width 0.5) (layer F.Cu) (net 18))
 (segment (start 24.19 18) (end 21.285 18) (width 0.5) (layer F.Cu) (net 13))
 (segment (start 21.285 18) (end 17.785 21.5) (width 0.5) (layer F.Cu) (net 13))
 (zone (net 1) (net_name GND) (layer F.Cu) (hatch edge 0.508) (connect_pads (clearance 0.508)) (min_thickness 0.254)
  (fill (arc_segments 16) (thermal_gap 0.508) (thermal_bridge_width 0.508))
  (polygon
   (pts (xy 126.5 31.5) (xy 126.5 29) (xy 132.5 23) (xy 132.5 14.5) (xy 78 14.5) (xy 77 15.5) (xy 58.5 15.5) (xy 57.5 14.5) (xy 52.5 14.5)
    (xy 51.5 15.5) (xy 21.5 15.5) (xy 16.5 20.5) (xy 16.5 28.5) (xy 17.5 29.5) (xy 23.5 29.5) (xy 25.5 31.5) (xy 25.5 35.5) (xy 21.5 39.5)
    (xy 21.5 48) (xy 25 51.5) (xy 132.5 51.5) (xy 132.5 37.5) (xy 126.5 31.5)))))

